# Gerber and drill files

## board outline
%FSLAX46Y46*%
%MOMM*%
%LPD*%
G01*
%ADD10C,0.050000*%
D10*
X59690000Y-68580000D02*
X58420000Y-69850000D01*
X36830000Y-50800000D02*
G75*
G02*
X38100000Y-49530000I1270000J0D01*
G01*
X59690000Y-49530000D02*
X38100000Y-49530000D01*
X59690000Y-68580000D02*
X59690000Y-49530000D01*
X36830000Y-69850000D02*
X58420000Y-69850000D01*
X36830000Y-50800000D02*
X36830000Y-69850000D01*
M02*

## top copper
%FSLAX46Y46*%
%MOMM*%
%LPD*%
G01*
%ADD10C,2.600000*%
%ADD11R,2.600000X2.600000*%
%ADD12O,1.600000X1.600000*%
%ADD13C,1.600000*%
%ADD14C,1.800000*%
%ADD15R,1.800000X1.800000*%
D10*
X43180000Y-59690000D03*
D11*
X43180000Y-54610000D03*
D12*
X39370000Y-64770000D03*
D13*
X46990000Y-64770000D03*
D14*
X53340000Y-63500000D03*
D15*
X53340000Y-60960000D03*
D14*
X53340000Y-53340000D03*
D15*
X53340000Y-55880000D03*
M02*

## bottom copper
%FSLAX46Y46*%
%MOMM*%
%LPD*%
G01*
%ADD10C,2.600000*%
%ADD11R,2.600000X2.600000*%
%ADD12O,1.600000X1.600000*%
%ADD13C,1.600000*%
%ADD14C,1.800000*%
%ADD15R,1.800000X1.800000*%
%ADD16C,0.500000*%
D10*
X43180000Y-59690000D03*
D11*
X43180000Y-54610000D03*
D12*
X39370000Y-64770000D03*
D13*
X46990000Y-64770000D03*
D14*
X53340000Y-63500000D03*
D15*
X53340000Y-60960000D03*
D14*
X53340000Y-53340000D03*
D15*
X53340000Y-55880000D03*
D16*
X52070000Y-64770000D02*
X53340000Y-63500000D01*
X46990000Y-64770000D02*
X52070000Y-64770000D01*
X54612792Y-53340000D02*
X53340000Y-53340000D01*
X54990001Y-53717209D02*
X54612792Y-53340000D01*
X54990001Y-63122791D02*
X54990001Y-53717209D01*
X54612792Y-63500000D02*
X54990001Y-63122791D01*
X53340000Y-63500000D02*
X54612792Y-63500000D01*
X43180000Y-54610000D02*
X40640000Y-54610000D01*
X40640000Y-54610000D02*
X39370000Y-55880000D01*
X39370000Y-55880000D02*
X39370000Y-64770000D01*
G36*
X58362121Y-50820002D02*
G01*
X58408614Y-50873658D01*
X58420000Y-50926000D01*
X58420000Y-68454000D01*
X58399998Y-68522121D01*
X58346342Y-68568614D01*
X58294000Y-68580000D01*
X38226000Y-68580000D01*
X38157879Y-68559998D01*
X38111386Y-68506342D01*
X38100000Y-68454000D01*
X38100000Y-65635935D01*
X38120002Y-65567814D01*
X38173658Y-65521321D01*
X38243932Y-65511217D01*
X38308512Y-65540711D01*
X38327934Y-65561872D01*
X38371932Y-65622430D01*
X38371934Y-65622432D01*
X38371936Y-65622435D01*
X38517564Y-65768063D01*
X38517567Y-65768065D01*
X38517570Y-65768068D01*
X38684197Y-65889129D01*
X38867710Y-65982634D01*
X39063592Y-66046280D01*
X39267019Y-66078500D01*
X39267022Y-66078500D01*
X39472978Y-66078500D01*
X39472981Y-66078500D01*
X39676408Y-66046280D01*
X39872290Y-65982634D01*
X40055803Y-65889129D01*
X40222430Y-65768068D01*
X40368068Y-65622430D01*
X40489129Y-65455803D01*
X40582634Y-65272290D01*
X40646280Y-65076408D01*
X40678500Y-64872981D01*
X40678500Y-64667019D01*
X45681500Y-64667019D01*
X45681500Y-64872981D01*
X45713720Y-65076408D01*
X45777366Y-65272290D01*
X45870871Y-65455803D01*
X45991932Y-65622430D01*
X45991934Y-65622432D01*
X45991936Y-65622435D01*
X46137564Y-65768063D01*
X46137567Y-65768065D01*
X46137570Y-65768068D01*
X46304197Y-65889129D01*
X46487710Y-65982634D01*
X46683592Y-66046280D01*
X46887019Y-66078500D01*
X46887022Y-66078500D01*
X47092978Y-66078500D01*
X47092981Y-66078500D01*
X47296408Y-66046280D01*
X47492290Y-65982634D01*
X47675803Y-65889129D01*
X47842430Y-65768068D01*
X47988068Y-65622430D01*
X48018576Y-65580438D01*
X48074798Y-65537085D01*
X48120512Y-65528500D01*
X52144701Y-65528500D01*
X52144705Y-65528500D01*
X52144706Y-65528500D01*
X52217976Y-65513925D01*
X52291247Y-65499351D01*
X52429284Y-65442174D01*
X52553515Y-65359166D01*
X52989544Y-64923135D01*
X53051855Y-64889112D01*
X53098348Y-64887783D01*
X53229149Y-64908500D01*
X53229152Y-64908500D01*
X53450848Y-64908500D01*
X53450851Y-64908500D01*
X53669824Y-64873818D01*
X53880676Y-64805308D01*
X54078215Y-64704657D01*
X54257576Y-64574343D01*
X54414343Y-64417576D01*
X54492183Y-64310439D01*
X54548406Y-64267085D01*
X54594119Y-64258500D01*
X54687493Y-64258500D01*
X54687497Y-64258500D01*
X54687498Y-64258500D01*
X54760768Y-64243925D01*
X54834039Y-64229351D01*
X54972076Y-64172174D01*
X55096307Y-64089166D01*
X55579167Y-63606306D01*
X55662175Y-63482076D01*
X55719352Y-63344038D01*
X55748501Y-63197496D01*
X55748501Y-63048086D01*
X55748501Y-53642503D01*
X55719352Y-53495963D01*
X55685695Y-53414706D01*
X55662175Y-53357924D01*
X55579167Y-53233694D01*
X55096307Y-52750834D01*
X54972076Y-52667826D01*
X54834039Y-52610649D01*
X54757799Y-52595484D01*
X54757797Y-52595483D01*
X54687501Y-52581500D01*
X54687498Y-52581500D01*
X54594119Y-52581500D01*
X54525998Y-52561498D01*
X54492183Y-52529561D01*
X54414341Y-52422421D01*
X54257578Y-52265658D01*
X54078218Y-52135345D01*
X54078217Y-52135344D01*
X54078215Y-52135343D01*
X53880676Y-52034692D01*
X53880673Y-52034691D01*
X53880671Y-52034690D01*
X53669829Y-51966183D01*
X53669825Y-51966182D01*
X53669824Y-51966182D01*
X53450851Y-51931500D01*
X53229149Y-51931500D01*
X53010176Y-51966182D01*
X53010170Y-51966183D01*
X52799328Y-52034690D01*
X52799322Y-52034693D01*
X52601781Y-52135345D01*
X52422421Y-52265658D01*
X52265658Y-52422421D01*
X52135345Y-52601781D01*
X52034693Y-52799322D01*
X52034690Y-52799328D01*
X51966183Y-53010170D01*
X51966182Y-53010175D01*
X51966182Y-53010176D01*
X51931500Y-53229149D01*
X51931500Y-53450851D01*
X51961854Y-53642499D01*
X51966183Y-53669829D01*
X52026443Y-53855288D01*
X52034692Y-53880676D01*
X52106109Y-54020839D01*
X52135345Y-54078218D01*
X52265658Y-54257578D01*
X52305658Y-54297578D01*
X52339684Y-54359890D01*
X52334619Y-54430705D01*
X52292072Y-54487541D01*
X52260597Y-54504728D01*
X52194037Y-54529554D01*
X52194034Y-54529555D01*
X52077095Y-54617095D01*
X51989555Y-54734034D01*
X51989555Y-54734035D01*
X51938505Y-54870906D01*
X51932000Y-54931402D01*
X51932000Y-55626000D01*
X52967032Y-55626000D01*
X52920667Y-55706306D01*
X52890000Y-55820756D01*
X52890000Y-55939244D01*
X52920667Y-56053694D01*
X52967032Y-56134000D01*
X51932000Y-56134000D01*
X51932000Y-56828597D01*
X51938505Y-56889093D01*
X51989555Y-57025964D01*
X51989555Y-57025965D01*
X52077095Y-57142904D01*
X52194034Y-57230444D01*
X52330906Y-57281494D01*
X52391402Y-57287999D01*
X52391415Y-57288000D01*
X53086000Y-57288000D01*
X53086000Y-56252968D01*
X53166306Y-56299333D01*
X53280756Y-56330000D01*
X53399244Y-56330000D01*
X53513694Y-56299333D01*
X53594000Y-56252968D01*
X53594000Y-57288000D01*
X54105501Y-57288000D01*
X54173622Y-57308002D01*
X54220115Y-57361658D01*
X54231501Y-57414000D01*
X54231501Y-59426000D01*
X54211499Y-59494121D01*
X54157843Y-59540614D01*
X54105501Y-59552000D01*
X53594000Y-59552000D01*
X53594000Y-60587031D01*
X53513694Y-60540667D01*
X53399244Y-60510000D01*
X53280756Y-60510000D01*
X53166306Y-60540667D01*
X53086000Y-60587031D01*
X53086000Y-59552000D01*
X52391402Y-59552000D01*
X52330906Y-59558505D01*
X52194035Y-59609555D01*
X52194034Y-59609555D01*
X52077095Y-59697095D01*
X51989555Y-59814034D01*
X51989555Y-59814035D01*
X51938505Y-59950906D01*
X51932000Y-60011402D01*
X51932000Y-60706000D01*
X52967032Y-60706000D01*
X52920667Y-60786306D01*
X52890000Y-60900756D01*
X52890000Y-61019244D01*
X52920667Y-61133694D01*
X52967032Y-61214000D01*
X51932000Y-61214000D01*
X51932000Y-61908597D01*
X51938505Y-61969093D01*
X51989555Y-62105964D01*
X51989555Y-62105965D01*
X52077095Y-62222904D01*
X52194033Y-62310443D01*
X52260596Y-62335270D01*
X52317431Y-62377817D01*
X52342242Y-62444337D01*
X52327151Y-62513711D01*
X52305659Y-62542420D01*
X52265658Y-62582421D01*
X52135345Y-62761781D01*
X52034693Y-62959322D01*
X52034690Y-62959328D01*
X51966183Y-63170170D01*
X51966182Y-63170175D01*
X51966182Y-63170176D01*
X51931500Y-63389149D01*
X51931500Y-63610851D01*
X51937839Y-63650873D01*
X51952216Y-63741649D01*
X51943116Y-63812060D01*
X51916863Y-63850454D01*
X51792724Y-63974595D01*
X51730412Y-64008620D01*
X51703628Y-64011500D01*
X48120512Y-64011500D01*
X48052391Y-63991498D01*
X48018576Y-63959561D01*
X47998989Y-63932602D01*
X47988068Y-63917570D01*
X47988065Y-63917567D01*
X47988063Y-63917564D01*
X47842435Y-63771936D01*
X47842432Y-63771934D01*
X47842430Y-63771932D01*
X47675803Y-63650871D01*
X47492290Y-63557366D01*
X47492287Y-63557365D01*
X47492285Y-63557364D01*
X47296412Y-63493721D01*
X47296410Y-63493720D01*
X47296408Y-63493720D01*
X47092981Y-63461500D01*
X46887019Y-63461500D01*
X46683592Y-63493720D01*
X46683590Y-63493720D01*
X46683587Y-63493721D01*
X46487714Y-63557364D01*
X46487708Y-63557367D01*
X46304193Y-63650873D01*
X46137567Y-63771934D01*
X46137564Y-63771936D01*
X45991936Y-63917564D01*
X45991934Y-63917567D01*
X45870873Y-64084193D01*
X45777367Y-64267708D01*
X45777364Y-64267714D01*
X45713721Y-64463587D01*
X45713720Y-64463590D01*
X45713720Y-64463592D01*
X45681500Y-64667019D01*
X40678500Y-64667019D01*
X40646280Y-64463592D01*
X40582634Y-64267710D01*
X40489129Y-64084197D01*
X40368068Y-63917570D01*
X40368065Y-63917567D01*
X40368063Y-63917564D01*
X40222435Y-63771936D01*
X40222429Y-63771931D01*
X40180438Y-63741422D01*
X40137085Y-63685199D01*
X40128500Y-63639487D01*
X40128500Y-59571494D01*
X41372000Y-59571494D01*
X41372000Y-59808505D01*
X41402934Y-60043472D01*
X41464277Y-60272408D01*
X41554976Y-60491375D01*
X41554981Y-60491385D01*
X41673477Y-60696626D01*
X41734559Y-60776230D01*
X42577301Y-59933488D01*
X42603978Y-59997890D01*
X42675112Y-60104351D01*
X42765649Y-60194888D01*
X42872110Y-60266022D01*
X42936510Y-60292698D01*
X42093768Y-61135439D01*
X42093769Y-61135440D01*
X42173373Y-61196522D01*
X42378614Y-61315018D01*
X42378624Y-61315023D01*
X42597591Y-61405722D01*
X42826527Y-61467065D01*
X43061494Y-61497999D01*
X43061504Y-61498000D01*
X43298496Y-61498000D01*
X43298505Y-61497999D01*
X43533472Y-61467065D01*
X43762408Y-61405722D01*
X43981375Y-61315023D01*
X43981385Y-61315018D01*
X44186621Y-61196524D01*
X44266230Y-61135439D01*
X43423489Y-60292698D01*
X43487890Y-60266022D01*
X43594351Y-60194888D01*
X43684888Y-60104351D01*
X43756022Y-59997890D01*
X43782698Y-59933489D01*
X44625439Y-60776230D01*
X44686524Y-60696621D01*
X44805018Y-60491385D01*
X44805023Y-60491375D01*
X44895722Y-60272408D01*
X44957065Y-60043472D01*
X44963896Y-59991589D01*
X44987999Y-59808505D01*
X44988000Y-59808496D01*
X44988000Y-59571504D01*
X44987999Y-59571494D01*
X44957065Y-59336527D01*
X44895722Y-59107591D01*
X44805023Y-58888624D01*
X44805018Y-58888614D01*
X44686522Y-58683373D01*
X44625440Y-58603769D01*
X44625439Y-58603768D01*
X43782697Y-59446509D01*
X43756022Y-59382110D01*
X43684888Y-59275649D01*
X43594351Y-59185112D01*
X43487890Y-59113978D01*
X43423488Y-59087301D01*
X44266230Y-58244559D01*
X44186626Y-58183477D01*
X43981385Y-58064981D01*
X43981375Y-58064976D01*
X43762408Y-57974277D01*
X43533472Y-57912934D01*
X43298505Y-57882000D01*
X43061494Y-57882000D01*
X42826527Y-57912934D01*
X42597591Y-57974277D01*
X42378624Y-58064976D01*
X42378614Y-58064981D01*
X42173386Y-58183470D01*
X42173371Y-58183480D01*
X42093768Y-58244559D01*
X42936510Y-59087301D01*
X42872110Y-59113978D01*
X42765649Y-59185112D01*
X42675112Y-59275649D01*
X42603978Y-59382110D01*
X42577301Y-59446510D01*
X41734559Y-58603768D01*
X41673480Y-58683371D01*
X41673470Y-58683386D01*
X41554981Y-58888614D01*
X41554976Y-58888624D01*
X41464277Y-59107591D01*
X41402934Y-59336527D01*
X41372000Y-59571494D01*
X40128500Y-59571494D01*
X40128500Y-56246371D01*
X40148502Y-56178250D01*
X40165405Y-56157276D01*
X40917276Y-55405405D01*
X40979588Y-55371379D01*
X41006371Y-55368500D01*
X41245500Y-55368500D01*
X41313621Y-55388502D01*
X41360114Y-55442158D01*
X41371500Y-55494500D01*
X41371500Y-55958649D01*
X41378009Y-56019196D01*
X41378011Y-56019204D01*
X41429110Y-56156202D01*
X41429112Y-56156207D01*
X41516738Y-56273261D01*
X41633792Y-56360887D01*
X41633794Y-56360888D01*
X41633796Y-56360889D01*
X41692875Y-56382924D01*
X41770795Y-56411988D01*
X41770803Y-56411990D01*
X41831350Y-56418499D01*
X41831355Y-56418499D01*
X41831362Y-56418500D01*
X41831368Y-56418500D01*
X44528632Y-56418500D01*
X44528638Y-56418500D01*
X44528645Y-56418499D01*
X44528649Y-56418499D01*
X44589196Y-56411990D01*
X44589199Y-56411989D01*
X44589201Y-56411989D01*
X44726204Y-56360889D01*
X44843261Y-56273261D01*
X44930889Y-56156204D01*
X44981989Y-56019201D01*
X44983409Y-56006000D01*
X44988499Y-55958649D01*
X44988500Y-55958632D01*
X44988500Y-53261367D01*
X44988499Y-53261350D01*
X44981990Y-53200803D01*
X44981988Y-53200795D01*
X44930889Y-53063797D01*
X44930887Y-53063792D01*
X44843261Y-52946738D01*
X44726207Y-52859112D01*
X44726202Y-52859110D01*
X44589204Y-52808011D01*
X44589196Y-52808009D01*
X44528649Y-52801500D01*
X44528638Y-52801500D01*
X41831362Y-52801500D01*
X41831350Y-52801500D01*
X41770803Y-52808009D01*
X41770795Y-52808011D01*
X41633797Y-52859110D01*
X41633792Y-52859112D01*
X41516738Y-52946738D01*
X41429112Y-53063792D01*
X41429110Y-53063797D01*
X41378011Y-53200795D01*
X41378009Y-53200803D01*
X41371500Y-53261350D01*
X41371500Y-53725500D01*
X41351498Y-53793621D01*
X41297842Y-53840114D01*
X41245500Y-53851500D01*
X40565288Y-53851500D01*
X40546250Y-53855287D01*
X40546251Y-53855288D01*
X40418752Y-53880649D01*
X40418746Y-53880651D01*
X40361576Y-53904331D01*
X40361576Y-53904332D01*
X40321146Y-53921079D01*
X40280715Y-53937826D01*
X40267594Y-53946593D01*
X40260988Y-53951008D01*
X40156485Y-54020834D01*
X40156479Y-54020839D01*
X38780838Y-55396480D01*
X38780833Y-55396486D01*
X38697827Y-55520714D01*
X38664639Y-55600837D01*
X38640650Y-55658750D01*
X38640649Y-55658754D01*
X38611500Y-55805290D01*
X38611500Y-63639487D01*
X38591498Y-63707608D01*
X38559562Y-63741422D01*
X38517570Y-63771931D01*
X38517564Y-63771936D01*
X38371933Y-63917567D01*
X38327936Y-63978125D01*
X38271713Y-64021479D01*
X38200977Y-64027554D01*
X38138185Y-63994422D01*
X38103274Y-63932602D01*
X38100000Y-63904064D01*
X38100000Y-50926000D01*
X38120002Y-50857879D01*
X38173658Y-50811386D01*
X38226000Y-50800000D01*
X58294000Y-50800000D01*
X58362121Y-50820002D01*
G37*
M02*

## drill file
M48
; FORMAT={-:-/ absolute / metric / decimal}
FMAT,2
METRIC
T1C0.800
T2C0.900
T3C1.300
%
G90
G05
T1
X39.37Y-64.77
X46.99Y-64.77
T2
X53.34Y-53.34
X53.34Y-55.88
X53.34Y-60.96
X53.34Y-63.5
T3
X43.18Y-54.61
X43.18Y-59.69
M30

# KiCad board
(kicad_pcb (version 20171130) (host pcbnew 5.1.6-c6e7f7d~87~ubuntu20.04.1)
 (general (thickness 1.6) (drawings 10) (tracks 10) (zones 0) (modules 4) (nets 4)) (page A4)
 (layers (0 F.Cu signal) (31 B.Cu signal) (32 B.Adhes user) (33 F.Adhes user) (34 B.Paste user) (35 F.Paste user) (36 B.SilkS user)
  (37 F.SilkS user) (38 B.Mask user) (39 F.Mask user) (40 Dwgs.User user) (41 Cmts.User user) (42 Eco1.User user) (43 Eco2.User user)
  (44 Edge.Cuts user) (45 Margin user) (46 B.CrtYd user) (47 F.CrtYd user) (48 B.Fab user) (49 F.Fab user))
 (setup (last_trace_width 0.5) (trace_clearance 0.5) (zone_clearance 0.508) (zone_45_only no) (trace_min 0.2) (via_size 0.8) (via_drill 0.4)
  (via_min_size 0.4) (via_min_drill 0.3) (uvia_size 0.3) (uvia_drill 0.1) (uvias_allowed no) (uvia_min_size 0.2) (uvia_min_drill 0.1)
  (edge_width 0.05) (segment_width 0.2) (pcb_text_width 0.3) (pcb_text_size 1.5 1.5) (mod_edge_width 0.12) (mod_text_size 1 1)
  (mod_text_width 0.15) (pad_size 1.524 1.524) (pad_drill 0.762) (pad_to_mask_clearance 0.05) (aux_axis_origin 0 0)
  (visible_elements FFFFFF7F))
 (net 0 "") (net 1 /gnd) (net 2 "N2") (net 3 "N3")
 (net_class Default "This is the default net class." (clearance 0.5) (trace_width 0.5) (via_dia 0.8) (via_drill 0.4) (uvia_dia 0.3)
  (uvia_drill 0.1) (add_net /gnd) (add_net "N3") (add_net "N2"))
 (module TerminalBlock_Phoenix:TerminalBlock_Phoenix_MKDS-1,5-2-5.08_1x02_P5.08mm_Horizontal (layer F.Cu) (at 43.18 54.61 270)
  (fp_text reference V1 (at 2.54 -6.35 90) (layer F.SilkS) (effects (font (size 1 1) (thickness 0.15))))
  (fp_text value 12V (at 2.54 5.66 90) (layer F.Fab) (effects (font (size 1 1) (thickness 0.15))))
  (pad 2 thru_hole circle (at 5.08 0 270) (size 2.6 2.6) (drill 1.3) (layers *.Cu *.Mask) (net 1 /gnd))
  (pad 1 thru_hole rect (at 0 0 270) (size 2.6 2.6) (drill 1.3) (layers *.Cu *.Mask) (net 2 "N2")))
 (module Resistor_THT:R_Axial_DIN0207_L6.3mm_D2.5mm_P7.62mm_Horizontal (layer F.Cu) (at 46.99 64.77 180)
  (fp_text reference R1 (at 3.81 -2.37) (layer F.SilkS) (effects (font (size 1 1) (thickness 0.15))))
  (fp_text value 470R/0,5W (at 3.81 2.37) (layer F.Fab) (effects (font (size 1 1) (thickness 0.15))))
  (pad 2 thru_hole oval (at 7.62 0 180) (size 1.6 1.6) (drill 0.8) (layers *.Cu *.Mask) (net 2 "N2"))
  (pad 1 thru_hole circle (at 0 0 180) (size 1.6 1.6) (drill 0.8) (layers *.Cu *.Mask) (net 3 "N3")))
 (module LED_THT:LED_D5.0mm (layer F.Cu) (at 53.34 60.96 270)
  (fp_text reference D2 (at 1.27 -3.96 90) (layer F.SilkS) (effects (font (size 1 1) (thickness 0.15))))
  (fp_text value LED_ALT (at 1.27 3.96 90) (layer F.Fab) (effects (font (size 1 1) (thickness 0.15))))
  (pad 2 thru_hole circle (at 2.54 0 270) (size 1.8 1.8) (drill 0.9) (layers *.Cu *.Mask) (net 3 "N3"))
  (pad 1 thru_hole rect (at 0 0 270) (size 1.8 1.8) (drill 0.9) (layers *.Cu *.Mask) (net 1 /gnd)))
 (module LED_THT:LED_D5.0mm (layer F.Cu) (at 53.34 55.88 90)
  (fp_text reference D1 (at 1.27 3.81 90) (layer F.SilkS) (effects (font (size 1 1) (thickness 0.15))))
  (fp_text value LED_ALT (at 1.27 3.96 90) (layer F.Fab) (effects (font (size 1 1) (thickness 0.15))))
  (pad 2 thru_hole circle (at 2.54 0 90) (size 1.8 1.8) (drill 0.9) (layers *.Cu *.Mask) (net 3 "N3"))
  (pad 1 thru_hole rect (at 0 0 90) (size 1.8 1.8) (drill 0.9) (layers *.Cu *.Mask) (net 1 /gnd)))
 (gr_line (start 59.69 68.58) (end 58.42 69.85) (layer Edge.Cuts) (width 0.05))
 (gr_arc (start 38.1 50.8) (end 38.1 49.53) (angle -90) (layer Edge.Cuts) (width 0.05))
 (gr_line (start 59.69 49.53) (end 38.1 49.53) (layer Edge.Cuts) (width 0.05))
 (gr_line (start 59.69 68.58) (end 59.69 49.53) (layer Edge.Cuts) (width 0.05))
 (gr_line (start 36.83 69.85) (end 58.42 69.85) (layer Edge.Cuts) (width 0.05))
 (gr_line (start 36.83 50.8) (end 36.83 69.85) (layer Edge.Cuts) (width 0.05))
 (segment (start 52.07 64.77) (end 53.34 63.5) (width 0.5) (layer B.Cu) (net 3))
 (segment (start 46.99 64.77) (end 52.07 64.77) (width 0.5) (layer B.Cu) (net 3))
 (segment (start 54.612792 53.34) (end 53.34 53.34) (width 0.5) (layer B.Cu) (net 3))
 (segment (start 54.990001 53.717209) (end 54.612792 53.34) (width 0.5) (layer B.Cu) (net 3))
 (segment (start 54.990001 63.122791) (end 54.990001 53.717209) (width 0.5) (layer B.Cu) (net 3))
 (segment (start 54.612792 63.5) (end 54.990001 63.122791) (width 0.5) (layer B.Cu) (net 3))
 (segment (start 53.34 63.5) (end 54.612792 63.5) (width 0.5) (layer B.Cu) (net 3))
 (segment (start 43.18 54.61) (end 40.64 54.61) (width 0.5) (layer B.Cu) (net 2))
 (segment (start 40.64 54.61) (end 39.37 55.88) (width 0.5) (layer B.Cu) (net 2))
 (segment (start 39.37 55.88) (end 39.37 64.77) (width 0.5) (layer B.Cu) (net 2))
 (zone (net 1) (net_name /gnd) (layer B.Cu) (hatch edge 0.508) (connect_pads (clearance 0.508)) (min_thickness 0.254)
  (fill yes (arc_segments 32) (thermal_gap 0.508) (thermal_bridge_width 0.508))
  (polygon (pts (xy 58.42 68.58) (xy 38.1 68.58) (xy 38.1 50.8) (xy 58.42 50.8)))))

